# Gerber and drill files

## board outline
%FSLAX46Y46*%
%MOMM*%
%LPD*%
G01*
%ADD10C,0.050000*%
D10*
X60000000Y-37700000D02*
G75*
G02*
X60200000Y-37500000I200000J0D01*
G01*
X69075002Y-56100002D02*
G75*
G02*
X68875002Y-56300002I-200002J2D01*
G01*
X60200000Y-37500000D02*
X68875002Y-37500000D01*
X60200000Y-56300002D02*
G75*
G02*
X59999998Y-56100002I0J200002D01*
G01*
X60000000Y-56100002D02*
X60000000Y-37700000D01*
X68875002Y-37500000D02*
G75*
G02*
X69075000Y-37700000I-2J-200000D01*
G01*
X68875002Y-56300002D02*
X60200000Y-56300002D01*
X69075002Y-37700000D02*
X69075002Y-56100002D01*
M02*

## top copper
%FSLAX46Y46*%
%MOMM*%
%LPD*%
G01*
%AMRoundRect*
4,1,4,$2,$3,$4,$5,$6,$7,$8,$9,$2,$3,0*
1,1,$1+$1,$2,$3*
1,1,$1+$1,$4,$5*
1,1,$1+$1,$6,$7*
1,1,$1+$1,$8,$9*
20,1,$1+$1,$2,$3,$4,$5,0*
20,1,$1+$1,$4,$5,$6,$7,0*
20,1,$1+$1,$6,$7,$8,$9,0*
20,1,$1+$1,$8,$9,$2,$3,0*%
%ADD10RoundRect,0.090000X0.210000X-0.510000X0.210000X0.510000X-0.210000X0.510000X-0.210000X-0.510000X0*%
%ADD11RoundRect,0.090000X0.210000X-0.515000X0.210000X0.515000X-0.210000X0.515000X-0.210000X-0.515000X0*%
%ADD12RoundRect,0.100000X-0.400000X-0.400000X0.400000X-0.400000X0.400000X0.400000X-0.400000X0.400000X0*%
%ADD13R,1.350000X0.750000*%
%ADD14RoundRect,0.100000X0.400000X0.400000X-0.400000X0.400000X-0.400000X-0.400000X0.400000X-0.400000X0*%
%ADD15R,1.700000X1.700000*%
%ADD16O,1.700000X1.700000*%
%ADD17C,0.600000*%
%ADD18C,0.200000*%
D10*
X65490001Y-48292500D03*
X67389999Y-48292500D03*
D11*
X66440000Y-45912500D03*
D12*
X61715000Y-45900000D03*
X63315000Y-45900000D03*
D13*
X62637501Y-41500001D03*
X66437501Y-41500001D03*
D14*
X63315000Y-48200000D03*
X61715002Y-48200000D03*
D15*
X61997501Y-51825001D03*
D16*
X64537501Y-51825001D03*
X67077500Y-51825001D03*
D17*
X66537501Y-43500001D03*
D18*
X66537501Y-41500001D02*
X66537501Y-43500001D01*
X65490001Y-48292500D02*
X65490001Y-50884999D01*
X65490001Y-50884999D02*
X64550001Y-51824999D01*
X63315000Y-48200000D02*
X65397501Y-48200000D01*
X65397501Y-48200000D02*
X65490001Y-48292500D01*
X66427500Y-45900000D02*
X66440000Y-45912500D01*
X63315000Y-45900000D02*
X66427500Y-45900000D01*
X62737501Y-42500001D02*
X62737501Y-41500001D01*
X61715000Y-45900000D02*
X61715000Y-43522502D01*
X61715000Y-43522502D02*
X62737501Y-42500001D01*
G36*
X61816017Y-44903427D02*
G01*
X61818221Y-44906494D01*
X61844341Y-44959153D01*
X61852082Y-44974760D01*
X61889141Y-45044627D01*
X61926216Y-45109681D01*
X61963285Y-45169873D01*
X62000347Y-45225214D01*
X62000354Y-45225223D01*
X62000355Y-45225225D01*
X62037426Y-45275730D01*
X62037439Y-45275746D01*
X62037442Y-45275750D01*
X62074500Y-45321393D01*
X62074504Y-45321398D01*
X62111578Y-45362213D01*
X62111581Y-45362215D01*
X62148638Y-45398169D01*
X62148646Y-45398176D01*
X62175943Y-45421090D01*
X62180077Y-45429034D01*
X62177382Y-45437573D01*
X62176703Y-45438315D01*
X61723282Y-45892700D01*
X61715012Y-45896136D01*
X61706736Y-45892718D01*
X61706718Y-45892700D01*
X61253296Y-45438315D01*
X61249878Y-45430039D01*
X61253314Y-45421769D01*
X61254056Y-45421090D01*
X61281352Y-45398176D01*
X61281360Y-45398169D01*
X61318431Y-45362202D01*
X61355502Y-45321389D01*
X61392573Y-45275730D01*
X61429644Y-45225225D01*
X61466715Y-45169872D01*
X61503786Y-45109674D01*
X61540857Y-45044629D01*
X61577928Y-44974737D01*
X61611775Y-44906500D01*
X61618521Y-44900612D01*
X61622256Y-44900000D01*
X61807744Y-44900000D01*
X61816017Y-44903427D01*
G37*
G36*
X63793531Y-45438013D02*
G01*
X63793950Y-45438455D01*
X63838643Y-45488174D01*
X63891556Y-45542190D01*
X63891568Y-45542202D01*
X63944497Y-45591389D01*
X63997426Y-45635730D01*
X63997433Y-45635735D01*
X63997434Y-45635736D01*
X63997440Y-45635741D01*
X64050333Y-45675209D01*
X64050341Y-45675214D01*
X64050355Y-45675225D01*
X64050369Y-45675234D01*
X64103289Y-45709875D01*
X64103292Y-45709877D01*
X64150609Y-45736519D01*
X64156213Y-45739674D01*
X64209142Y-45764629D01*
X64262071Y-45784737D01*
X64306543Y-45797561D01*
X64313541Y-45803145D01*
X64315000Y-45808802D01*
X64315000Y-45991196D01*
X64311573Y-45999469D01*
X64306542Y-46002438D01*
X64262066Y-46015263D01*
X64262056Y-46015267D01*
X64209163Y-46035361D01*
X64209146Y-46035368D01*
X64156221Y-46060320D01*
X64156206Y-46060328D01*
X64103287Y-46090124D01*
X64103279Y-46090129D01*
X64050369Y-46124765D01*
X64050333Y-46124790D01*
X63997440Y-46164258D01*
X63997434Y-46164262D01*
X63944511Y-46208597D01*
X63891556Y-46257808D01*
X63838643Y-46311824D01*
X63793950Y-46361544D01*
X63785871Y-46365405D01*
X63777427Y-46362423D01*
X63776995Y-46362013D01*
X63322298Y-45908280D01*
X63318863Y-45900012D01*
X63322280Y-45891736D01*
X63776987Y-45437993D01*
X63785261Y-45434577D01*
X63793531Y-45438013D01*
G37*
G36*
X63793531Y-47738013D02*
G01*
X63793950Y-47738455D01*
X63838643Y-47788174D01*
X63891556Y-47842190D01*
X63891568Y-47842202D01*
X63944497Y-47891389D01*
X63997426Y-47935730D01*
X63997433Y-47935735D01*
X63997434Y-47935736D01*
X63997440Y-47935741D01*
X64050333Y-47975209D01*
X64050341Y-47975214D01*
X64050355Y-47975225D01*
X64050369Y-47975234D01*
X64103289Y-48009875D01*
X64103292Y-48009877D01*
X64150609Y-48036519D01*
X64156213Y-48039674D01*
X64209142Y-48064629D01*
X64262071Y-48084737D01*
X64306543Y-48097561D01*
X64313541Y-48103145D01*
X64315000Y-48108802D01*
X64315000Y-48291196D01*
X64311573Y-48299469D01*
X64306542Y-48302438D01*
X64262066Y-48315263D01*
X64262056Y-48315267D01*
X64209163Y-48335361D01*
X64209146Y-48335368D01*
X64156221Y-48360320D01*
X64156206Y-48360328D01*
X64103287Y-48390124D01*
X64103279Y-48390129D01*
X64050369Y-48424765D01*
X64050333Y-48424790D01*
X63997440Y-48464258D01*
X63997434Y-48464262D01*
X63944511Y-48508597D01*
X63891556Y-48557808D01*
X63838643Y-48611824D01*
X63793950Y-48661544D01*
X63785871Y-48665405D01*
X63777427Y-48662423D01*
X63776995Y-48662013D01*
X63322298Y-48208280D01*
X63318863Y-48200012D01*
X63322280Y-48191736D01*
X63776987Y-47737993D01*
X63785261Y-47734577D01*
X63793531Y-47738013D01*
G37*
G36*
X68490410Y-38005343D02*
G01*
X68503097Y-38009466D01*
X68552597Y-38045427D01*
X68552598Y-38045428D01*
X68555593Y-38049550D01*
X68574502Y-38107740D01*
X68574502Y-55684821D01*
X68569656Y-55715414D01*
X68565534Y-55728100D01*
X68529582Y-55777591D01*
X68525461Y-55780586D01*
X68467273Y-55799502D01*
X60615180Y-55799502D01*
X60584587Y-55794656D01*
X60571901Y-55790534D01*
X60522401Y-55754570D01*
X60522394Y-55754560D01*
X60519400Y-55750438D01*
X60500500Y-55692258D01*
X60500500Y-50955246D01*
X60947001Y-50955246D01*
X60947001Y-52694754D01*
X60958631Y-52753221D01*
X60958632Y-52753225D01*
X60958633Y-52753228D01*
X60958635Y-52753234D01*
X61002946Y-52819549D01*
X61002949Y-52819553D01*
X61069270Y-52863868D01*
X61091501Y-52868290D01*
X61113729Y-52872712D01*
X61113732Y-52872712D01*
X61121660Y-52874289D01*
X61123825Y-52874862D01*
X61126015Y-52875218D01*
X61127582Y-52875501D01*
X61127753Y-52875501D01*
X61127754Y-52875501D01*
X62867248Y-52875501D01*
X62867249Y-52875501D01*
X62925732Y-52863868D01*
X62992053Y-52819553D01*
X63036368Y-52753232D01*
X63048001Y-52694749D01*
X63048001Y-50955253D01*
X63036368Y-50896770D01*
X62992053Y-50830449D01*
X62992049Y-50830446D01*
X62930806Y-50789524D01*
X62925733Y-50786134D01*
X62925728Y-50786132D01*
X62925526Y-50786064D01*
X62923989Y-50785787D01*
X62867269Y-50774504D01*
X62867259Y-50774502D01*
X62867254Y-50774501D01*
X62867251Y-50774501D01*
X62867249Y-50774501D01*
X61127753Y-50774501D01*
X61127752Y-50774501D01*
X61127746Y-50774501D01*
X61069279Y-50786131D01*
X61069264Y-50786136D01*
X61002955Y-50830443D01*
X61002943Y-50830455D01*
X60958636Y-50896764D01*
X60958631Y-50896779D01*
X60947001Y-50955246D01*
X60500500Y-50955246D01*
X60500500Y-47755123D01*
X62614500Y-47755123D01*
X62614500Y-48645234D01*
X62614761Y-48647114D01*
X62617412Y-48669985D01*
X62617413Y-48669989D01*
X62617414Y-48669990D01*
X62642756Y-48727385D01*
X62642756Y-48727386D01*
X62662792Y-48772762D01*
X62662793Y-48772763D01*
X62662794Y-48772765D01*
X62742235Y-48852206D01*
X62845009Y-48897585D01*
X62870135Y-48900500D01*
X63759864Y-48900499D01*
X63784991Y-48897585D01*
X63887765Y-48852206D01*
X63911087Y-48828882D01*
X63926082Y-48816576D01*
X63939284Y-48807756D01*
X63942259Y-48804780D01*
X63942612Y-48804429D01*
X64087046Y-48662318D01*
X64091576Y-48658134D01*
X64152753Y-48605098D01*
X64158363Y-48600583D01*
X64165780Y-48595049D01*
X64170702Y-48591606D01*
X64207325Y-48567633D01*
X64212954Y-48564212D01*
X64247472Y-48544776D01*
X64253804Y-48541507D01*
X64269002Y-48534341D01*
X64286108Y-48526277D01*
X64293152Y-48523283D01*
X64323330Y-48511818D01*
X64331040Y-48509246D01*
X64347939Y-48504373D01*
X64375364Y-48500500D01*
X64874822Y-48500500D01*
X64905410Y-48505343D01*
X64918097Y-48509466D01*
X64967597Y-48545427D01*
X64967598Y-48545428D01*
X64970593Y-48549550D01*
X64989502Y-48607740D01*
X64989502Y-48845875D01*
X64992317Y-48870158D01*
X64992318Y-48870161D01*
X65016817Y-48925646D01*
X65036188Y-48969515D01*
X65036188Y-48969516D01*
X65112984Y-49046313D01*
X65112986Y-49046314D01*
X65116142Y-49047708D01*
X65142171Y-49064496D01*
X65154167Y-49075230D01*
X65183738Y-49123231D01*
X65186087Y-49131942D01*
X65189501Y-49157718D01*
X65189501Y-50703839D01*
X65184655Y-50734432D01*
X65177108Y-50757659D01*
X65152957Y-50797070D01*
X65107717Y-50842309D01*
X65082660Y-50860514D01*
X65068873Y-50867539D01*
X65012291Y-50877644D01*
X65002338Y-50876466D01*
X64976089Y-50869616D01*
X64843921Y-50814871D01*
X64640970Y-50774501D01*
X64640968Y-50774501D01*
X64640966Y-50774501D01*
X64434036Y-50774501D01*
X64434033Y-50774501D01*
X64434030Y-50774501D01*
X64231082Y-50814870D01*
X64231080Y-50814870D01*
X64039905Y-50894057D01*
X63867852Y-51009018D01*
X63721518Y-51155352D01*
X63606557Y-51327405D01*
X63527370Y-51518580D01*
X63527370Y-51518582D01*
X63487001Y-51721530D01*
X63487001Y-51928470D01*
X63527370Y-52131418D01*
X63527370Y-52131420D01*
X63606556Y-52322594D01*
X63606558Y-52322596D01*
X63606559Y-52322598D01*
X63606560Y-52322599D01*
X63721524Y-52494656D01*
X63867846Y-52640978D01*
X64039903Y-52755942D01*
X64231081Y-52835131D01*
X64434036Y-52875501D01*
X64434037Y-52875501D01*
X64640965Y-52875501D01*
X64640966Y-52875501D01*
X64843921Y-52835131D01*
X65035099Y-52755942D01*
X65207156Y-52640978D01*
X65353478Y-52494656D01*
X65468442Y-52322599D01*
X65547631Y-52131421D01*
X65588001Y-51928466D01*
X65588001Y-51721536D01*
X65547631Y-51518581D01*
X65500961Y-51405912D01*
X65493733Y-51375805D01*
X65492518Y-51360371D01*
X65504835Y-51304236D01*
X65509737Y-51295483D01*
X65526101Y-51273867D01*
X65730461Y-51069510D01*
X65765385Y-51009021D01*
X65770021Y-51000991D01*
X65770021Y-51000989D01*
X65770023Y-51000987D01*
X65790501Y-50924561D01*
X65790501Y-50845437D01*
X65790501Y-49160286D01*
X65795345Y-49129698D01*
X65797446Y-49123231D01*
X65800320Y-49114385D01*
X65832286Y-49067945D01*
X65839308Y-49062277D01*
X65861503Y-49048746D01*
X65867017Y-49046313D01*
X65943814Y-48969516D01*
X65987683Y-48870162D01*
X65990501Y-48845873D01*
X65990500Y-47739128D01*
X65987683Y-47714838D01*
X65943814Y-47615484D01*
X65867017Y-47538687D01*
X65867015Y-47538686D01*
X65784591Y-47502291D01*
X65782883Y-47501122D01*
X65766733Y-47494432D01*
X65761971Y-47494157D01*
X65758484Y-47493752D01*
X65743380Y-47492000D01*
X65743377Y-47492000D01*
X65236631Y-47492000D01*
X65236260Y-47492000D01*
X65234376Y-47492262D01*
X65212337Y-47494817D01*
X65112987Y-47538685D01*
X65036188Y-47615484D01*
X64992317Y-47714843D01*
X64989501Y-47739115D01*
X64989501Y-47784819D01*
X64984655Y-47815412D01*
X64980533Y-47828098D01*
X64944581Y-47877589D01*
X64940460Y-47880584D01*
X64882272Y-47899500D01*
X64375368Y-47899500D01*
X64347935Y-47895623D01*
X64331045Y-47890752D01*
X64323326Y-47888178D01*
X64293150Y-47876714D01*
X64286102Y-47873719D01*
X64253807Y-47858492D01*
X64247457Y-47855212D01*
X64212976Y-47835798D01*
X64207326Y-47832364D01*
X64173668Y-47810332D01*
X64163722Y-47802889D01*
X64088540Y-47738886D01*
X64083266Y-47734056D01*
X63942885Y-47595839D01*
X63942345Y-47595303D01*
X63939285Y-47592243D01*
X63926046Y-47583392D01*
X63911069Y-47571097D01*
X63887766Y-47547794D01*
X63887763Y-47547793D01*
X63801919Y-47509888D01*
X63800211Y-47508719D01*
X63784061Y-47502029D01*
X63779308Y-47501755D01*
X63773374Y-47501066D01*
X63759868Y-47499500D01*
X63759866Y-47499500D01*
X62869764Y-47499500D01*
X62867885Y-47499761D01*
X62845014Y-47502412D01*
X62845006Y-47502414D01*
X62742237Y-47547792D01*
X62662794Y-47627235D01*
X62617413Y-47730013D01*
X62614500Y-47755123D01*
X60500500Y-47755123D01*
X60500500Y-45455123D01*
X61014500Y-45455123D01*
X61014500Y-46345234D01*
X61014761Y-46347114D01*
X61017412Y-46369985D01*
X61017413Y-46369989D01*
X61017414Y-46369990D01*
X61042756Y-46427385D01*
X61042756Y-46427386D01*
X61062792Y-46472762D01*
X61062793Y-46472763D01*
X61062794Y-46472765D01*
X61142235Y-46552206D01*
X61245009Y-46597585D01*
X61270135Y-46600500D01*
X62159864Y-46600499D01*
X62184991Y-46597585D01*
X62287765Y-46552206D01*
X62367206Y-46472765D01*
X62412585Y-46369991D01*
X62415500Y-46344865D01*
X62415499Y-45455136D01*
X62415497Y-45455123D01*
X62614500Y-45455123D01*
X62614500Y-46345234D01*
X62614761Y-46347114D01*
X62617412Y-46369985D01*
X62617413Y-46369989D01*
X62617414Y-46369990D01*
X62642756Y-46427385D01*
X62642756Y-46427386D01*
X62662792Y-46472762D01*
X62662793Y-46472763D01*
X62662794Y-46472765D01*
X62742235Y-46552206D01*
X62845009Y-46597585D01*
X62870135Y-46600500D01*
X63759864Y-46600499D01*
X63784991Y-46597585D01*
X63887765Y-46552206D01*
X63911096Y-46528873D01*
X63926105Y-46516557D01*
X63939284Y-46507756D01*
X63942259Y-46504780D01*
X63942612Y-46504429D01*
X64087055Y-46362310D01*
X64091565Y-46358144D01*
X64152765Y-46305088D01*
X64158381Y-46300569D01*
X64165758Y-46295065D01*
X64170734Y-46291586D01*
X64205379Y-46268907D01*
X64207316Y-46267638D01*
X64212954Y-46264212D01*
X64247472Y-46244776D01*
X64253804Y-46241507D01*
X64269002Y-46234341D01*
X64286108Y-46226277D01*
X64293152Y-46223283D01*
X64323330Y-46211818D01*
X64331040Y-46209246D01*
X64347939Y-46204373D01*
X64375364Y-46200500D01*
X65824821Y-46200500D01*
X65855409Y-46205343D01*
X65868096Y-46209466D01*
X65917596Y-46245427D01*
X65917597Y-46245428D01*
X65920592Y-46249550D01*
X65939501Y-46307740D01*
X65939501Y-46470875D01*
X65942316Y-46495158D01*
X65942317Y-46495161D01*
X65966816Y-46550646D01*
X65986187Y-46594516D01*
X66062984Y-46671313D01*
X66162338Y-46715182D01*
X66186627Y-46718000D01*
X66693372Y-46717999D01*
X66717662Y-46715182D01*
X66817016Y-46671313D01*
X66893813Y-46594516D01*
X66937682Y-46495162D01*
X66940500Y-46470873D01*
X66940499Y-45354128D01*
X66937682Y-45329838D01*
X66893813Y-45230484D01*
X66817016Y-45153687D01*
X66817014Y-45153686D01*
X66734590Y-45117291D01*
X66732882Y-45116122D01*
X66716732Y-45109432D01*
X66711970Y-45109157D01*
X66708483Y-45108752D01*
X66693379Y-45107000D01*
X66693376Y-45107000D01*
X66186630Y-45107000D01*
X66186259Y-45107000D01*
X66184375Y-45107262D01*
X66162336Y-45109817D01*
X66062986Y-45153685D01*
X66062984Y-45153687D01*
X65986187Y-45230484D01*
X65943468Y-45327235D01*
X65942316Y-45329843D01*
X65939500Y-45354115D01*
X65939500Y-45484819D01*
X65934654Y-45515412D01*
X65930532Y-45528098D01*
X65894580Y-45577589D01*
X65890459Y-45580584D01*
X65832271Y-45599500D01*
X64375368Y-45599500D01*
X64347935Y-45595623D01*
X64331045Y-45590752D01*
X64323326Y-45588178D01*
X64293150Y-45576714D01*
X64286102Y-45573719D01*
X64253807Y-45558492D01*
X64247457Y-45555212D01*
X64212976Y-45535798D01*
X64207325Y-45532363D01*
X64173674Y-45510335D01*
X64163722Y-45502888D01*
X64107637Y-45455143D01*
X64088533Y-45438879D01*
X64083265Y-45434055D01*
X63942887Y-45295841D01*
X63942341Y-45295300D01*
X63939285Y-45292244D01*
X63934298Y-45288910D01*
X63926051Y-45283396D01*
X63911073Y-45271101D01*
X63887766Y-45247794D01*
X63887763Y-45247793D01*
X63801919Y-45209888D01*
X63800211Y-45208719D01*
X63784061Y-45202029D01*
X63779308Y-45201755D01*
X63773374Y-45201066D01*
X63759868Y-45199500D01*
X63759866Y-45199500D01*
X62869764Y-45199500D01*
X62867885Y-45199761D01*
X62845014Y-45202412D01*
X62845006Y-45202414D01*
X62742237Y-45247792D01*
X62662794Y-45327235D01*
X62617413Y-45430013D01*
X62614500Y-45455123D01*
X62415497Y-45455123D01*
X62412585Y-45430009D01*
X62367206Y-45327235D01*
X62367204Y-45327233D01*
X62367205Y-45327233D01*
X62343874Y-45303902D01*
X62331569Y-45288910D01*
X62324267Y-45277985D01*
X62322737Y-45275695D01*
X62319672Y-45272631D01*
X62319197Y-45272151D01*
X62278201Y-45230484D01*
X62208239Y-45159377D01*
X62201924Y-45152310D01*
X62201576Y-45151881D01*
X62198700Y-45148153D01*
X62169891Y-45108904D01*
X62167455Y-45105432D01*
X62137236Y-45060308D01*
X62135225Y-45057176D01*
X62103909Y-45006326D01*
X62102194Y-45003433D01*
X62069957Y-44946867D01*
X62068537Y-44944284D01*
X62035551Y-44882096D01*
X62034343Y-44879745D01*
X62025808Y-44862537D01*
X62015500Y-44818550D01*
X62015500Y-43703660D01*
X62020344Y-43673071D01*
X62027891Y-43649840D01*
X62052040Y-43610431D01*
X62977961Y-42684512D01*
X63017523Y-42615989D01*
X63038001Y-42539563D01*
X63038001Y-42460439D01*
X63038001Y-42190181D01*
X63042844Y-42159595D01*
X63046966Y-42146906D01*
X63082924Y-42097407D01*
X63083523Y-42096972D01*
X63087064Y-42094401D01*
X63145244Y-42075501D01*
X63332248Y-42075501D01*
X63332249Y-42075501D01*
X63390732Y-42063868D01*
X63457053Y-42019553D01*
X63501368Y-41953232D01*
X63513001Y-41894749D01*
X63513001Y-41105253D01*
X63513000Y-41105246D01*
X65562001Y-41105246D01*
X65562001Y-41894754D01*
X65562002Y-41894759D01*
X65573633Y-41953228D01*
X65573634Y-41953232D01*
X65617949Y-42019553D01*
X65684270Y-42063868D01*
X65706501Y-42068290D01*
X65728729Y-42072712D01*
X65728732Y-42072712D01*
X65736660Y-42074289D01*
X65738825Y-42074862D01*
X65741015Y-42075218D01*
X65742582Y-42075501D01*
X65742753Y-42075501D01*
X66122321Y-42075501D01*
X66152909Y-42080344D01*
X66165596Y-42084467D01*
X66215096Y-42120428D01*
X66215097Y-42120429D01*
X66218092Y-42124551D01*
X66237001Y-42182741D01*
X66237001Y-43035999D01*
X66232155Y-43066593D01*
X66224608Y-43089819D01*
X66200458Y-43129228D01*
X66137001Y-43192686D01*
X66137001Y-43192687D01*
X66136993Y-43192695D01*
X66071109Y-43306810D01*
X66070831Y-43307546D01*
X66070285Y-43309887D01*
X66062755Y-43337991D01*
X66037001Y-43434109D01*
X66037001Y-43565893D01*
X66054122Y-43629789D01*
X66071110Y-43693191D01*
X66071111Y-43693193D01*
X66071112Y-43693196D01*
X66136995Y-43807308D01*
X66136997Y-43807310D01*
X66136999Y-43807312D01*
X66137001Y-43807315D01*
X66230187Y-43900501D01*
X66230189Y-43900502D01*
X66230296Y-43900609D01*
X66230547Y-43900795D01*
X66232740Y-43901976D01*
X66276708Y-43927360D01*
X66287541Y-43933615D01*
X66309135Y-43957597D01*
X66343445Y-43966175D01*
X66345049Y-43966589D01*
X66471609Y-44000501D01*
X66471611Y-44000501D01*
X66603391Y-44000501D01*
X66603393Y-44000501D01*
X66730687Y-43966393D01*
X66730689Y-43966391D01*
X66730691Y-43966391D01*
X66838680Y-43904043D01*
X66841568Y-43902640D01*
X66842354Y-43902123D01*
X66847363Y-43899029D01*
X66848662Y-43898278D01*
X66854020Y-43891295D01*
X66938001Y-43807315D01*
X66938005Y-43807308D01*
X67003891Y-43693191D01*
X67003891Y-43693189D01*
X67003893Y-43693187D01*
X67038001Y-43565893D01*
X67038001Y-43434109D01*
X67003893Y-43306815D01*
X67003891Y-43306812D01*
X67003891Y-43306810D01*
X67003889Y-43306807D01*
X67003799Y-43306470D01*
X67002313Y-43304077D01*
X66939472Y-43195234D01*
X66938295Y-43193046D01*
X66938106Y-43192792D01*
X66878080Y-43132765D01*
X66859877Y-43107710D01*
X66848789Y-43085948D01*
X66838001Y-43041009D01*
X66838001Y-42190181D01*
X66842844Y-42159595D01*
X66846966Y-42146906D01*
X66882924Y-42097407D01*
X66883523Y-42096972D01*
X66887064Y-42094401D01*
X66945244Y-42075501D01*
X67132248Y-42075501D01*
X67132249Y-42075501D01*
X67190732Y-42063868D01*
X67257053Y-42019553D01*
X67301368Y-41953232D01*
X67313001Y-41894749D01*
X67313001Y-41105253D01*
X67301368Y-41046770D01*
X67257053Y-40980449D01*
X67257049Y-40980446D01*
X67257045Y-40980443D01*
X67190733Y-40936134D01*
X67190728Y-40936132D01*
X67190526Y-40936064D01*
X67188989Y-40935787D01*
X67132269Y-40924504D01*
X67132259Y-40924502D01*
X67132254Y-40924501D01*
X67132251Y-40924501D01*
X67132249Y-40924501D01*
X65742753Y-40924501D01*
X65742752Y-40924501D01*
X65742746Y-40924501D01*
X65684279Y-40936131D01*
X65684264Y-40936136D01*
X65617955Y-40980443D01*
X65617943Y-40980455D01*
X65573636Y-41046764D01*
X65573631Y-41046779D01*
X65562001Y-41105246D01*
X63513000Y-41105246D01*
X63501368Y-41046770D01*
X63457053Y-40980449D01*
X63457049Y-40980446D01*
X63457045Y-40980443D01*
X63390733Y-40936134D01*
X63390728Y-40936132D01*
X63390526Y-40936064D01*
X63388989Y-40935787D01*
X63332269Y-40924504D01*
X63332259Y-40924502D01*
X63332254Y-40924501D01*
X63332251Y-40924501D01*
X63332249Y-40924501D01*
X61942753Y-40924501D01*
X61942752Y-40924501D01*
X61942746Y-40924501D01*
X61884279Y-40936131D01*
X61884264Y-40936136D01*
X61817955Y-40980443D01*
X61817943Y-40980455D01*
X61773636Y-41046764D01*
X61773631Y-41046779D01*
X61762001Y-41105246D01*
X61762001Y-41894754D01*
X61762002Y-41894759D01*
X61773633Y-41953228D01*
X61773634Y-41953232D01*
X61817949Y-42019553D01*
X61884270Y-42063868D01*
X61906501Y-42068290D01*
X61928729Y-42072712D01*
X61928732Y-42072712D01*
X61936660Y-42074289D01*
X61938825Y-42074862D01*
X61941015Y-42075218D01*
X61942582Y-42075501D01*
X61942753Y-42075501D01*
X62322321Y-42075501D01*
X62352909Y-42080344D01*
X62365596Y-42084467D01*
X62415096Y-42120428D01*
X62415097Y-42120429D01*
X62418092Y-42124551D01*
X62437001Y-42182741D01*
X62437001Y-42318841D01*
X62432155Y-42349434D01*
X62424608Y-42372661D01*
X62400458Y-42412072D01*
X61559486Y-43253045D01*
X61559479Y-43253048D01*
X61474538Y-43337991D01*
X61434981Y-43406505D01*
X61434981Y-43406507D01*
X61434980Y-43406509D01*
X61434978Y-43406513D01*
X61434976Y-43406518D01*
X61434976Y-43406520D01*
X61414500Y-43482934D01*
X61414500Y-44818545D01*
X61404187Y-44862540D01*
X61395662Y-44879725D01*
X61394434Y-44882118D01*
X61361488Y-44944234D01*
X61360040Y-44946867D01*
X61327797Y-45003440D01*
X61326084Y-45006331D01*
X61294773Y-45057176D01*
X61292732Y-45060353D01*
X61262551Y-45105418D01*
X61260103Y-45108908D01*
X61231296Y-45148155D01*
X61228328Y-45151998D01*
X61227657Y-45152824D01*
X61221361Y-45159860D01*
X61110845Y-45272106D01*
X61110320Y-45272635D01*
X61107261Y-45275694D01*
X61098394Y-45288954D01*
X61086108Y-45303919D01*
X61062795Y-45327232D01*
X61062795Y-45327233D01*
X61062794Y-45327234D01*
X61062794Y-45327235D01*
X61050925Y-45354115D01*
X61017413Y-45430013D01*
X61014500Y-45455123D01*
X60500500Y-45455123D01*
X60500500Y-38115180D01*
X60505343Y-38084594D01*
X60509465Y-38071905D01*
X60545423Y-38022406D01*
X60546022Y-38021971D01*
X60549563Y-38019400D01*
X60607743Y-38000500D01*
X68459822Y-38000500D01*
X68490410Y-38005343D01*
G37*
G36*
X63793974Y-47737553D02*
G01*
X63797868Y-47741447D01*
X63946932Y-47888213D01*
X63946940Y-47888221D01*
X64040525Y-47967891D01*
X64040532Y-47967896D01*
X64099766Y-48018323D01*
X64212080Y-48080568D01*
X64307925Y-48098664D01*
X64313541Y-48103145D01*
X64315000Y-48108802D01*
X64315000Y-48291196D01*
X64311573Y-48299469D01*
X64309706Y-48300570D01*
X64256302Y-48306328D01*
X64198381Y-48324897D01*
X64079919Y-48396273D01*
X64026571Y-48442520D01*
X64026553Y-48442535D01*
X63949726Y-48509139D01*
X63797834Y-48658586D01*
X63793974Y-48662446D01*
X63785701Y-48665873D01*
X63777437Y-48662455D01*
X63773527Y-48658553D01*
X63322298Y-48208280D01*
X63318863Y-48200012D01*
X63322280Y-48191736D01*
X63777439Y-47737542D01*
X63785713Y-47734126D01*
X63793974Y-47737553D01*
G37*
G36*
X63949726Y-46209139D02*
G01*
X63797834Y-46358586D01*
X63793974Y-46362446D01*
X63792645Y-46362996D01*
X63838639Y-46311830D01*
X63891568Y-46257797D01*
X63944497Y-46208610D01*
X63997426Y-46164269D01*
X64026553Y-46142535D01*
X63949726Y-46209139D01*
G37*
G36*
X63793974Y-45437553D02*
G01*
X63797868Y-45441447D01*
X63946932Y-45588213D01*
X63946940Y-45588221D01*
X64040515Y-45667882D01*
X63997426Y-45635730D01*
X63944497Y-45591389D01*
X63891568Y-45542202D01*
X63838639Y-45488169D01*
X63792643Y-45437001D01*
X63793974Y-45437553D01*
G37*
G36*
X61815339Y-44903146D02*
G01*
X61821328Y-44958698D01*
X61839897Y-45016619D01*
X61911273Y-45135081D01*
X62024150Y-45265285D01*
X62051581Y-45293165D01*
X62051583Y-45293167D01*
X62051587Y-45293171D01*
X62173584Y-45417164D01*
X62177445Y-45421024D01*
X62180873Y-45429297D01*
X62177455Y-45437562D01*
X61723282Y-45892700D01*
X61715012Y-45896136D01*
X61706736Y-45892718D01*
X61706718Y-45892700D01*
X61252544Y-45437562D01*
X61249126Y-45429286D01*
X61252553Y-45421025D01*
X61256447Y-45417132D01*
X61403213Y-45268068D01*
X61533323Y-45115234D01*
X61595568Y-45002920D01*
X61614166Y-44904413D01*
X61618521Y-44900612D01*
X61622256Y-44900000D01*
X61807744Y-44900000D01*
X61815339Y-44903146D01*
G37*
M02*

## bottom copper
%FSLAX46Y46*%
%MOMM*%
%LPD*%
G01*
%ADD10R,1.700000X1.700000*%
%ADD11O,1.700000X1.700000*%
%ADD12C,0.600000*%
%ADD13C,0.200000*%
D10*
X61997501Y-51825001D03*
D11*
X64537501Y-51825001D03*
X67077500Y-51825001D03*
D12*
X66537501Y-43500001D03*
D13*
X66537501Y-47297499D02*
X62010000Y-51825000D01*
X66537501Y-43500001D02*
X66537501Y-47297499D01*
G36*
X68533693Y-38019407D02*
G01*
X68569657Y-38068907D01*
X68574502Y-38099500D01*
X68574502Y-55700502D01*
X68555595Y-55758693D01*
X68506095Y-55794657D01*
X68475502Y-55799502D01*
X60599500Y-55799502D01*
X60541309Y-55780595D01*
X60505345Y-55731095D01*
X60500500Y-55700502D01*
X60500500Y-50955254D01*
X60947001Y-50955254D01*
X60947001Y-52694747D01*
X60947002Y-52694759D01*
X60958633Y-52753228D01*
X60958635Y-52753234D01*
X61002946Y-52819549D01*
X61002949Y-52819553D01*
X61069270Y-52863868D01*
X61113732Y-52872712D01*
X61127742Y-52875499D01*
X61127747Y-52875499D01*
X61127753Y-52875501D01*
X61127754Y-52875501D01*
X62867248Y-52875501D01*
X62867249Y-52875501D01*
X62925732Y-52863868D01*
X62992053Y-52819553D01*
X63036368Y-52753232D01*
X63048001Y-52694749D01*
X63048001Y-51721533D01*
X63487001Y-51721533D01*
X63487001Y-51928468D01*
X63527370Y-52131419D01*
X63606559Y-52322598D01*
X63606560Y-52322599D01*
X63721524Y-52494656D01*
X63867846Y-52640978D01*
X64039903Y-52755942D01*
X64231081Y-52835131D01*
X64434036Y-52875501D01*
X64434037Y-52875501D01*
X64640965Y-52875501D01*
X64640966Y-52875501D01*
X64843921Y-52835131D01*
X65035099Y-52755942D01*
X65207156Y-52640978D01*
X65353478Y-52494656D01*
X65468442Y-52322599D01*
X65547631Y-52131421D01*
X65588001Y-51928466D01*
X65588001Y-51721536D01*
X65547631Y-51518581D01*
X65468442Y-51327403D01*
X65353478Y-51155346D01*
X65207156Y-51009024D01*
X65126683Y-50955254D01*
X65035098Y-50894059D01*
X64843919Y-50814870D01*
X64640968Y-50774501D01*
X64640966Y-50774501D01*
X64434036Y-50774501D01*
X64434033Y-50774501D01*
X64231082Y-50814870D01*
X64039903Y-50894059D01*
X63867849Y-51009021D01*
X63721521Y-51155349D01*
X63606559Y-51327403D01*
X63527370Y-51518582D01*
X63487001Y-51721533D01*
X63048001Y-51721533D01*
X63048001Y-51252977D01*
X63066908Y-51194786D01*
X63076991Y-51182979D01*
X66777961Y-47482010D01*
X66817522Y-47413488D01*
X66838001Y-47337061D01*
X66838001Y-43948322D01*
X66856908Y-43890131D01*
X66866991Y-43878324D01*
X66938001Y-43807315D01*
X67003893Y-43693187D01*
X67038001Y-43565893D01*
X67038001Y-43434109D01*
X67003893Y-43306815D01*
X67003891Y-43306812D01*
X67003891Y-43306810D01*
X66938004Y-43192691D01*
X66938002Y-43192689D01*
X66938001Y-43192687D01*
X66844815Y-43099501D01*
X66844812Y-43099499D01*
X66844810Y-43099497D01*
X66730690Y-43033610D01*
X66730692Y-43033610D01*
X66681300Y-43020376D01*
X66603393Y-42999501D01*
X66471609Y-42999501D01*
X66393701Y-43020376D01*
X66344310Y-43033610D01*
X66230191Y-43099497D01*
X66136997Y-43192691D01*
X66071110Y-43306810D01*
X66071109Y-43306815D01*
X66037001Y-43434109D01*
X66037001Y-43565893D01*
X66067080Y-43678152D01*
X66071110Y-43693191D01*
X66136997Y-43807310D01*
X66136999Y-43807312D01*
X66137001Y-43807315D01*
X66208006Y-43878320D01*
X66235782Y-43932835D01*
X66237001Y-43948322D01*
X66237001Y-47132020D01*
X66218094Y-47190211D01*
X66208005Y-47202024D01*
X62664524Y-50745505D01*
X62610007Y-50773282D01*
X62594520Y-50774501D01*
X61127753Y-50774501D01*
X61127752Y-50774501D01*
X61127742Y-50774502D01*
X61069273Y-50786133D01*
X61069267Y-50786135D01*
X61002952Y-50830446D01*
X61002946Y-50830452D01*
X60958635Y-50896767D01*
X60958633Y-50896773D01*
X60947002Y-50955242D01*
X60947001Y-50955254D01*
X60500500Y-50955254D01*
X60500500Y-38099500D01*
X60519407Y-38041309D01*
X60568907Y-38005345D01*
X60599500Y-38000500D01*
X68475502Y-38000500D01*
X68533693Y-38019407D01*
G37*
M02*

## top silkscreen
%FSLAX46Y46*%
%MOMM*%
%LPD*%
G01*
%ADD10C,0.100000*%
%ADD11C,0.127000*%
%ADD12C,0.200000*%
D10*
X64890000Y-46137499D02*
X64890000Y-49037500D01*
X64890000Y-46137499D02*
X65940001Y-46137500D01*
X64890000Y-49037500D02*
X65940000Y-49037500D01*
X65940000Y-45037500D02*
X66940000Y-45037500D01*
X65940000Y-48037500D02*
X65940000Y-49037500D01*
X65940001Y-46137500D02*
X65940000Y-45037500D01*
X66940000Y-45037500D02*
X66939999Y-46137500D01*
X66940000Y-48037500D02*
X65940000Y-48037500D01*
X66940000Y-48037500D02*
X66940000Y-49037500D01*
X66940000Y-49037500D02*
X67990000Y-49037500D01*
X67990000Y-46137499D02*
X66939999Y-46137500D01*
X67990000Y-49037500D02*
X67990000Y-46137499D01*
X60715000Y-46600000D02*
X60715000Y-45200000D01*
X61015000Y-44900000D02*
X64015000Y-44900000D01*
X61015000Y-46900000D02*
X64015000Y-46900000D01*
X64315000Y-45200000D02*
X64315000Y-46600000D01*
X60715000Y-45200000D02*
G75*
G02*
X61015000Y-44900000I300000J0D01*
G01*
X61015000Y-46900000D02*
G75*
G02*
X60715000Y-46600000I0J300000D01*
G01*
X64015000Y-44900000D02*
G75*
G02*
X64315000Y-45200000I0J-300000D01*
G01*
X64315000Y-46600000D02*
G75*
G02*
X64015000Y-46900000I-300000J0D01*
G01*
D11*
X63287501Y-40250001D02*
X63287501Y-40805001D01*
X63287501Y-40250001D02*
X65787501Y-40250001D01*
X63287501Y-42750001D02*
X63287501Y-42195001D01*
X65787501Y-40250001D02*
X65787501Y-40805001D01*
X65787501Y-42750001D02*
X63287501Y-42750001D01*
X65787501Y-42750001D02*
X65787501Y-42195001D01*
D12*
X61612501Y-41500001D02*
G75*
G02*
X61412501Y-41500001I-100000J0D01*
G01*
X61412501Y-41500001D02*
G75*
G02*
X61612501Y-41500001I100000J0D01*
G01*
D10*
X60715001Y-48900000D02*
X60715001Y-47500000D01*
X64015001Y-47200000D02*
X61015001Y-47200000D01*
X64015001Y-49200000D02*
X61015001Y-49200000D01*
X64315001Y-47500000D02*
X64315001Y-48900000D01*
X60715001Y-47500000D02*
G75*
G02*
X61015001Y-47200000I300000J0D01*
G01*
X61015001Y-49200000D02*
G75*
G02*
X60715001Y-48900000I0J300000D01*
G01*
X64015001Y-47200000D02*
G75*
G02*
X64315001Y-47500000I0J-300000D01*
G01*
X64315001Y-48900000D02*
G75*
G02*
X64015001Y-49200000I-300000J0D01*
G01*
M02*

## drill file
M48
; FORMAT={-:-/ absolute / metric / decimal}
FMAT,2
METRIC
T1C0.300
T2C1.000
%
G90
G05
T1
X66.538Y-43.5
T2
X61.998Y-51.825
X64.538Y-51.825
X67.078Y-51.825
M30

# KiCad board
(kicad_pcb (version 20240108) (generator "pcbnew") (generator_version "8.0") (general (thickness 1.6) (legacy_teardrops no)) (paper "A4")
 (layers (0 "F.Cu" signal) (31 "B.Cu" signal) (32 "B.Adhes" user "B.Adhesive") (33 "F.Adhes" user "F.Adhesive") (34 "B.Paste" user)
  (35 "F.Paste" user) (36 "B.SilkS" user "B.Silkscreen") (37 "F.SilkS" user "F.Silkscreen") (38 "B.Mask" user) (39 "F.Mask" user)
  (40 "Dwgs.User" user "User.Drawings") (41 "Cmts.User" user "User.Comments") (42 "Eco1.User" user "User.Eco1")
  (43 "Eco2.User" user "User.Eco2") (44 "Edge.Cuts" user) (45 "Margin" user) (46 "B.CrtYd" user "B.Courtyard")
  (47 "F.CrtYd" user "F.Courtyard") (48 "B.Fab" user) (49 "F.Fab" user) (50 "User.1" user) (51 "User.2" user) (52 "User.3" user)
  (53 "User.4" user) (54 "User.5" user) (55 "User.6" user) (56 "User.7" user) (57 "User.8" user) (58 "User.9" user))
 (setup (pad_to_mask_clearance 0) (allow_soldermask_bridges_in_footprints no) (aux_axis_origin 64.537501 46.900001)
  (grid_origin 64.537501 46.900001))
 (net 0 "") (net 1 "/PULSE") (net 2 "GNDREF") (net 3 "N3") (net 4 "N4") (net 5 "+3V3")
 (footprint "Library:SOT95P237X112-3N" (layer "F.Cu") (at 66.44 47.0375 90)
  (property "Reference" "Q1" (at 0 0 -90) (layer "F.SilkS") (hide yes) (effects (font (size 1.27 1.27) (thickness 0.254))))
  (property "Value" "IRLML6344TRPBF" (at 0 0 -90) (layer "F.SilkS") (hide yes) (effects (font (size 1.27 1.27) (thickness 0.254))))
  (fp_line (start 0.900001 -1.55) (end -2 -1.55) (stroke (width 0.1) (type solid)) (layer "F.SilkS"))
  (fp_line (start 0.900001 -1.55) (end 0.9 -0.499999) (stroke (width 0.1) (type default)) (layer "F.SilkS"))
  (fp_line (start -2 -1.55) (end -2 -0.5) (stroke (width 0.1) (type default)) (layer "F.SilkS"))
  (fp_line (start 2 -0.5) (end 2 0.5) (stroke (width 0.1) (type default)) (layer "F.SilkS"))
  (fp_line (start -1 -0.5) (end -2 -0.5) (stroke (width 0.1) (type default)) (layer "F.SilkS"))
  (fp_line (start 0.9 -0.499999) (end 2 -0.5) (stroke (width 0.1) (type default)) (layer "F.SilkS"))
  (fp_line (start 2 0.5) (end 0.9 0.499999) (stroke (width 0.1) (type default)) (layer "F.SilkS"))
  (fp_line (start -1 0.5) (end -1 -0.5) (stroke (width 0.1) (type default)) (layer "F.SilkS"))
  (fp_line (start -1 0.5) (end -2 0.5) (stroke (width 0.1) (type default)) (layer "F.SilkS"))
  (fp_line (start -2 0.5) (end -2 1.55) (stroke (width 0.1) (type default)) (layer "F.SilkS"))
  (fp_line (start 0.900001 1.55) (end 0.9 0.499999) (stroke (width 0.1) (type default)) (layer "F.SilkS"))
  (fp_line (start -2 1.55) (end 0.900001 1.55) (stroke (width 0.1) (type solid)) (layer "F.SilkS"))
  (pad "1" smd roundrect (at -1.255 -0.949999 90) (size 1.2 0.6) (layers "F.Cu" "F.Paste" "F.Mask") (roundrect_rratio 0.15) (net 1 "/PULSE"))
  (pad "2" smd roundrect (at -1.255 0.949999 90) (size 1.2 0.6) (layers "F.Cu" "F.Paste" "F.Mask") (roundrect_rratio 0.15) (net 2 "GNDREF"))
  (pad "3" smd roundrect (at 1.125 0 90) (size 1.21 0.6) (layers "F.Cu" "F.Paste" "F.Mask") (roundrect_rratio 0.15) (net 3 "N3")))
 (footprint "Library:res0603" (layer "F.Cu") (at 62.515 45.9)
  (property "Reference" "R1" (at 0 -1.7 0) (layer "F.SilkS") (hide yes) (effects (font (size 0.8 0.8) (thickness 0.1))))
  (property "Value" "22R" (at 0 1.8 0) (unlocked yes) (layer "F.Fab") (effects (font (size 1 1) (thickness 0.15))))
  (fp_line (start -1.8 0.7) (end -1.8 -0.7) (stroke (width 0.1) (type default)) (layer "F.SilkS"))
  (fp_line (start -1.5 -1) (end 1.5 -1) (stroke (width 0.1) (type default)) (layer "F.SilkS"))
  (fp_line (start -1.5 1) (end 1.5 1) (stroke (width 0.1) (type default)) (layer "F.SilkS"))
  (fp_line (start 1.8 -0.7) (end 1.8 0.7) (stroke (width 0.1) (type default)) (layer "F.SilkS"))
  (fp_arc (start -1.8 -0.7) (mid -1.712132 -0.912132) (end -1.5 -1) (stroke (width 0.1) (type default)) (layer "F.SilkS"))
  (fp_arc (start -1.5 1) (mid -1.712132 0.912132) (end -1.8 0.7) (stroke (width 0.1) (type default)) (layer "F.SilkS"))
  (fp_arc (start 1.5 -1) (mid 1.712132 -0.912132) (end 1.8 -0.7) (stroke (width 0.1) (type default)) (layer "F.SilkS"))
  (fp_arc (start 1.8 0.7) (mid 1.712132 0.912132) (end 1.5 1) (stroke (width 0.1) (type default)) (layer "F.SilkS"))
  (pad "1" smd roundrect (at -0.8 0) (size 1 1) (layers "F.Cu" "F.Paste" "F.Mask") (roundrect_rratio 0.1) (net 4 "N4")
   (thermal_bridge_angle 45)
   (teardrops (best_length_ratio 0.5) (max_length 1) (best_width_ratio 1) (max_width 1) (curve_points 10) (filter_ratio 0.9) (enabled yes)
    (allow_two_segments yes) (prefer_zone_connections yes)))
  (pad "2" smd roundrect (at 0.8 0) (size 1 1) (layers "F.Cu" "F.Paste" "F.Mask") (roundrect_rratio 0.1) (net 3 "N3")
   (thermal_bridge_angle 45)
   (teardrops (best_length_ratio 0.5) (max_length 1) (best_width_ratio 1) (max_width 1) (curve_points 10) (filter_ratio 0.9) (enabled yes)
    (allow_two_segments yes) (prefer_zone_connections yes))))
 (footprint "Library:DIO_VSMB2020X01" (layer "F.Cu") (at 64.537501 41.500001)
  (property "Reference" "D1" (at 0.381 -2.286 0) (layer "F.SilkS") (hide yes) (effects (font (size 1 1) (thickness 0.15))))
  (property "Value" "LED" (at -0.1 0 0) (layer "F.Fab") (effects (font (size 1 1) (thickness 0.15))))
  (fp_line (start -1.25 -1.25) (end -1.25 -0.695) (stroke (width 0.127) (type solid)) (layer "F.SilkS"))
  (fp_line (start -1.25 -1.25) (end 1.25 -1.25) (stroke (width 0.127) (type solid)) (layer "F.SilkS"))
  (fp_line (start -1.25 1.25) (end -1.25 0.695) (stroke (width 0.127) (type solid)) (layer "F.SilkS"))
  (fp_line (start 1.25 -1.25) (end 1.25 -0.695) (stroke (width 0.127) (type solid)) (layer "F.SilkS"))
  (fp_line (start 1.25 1.25) (end -1.25 1.25) (stroke (width 0.127) (type solid)) (layer "F.SilkS"))
  (fp_line (start 1.25 1.25) (end 1.25 0.695) (stroke (width 0.127) (type solid)) (layer "F.SilkS"))
  (fp_circle (center -3.025 0) (end -2.925 0) (stroke (width 0.2) (type solid)) (fill none) (layer "F.SilkS"))
  (pad "1" smd rect (at -1.9 0) (size 1.35 0.75) (layers "F.Cu" "F.Paste" "F.Mask") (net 4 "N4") (solder_mask_margin 0.102))
  (pad "2" smd rect (at 1.9 0) (size 1.35 0.75) (layers "F.Cu" "F.Paste" "F.Mask") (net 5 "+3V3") (solder_mask_margin 0.102)))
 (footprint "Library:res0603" (layer "F.Cu") (at 62.515001 48.2 180)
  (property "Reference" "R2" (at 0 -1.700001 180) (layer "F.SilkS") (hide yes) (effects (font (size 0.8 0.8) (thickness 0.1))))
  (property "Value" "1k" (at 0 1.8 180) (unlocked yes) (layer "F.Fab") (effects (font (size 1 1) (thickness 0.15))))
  (fp_line (start 1.8 -0.7) (end 1.8 0.7) (stroke (width 0.1) (type default)) (layer "F.SilkS"))
  (fp_line (start -1.5 1) (end 1.5 1) (stroke (width 0.1) (type default)) (layer "F.SilkS"))
  (fp_line (start -1.5 -1) (end 1.5 -1) (stroke (width 0.1) (type default)) (layer "F.SilkS"))
  (fp_line (start -1.8 0.7) (end -1.8 -0.7) (stroke (width 0.1) (type default)) (layer "F.SilkS"))
  (fp_arc (start 1.8 0.7) (mid 1.712132 0.912132) (end 1.5 1) (stroke (width 0.1) (type default)) (layer "F.SilkS"))
  (fp_arc (start 1.5 -1) (mid 1.712132 -0.912132) (end 1.8 -0.7) (stroke (width 0.1) (type default)) (layer "F.SilkS"))
  (fp_arc (start -1.5 1) (mid -1.712132 0.912132) (end -1.8 0.7) (stroke (width 0.1) (type default)) (layer "F.SilkS"))
  (fp_arc (start -1.8 -0.7) (mid -1.712132 -0.912132) (end -1.5 -1) (stroke (width 0.1) (type default)) (layer "F.SilkS"))
  (pad "1" smd roundrect (at -0.799999 0 180) (size 1 1) (layers "F.Cu" "F.Paste" "F.Mask") (roundrect_rratio 0.1) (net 1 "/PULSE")
   (thermal_bridge_angle 45)
   (teardrops (best_length_ratio 0.5) (max_length 1) (best_width_ratio 1) (max_width 1) (curve_points 10) (filter_ratio 0.9) (enabled yes)
    (allow_two_segments yes) (prefer_zone_connections yes)))
  (pad "2" smd roundrect (at 0.799999 0 180) (size 1 1) (layers "F.Cu" "F.Paste" "F.Mask") (roundrect_rratio 0.1) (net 2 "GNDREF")
   (thermal_bridge_angle 45)
   (teardrops (best_length_ratio 0.5) (max_length 1) (best_width_ratio 1) (max_width 1) (curve_points 10) (filter_ratio 0.9) (enabled yes)
    (allow_two_segments yes) (prefer_zone_connections yes))))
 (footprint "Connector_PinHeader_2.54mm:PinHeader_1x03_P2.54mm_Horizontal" (layer "B.Cu") (at 61.997501 51.825001 -90)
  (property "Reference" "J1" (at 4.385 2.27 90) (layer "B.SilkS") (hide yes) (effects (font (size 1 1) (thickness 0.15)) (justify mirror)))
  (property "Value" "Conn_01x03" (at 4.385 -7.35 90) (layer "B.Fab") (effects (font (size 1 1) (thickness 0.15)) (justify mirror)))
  (pad "1" thru_hole rect (at 0 0 270) (size 1.7 1.7) (drill 1) (layers "*.Cu" "*.Mask") (remove_unused_layers no) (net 5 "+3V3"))
  (pad "2" thru_hole oval (at 0 -2.54 270) (size 1.7 1.7) (drill 1) (layers "*.Cu" "*.Mask") (remove_unused_layers no) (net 1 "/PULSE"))
  (pad "3" thru_hole oval (at 0 -5.079999 270) (size 1.7 1.7) (drill 1) (layers "*.Cu" "*.Mask") (remove_unused_layers no) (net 2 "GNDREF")))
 (gr_arc (start 60 37.7) (mid 60.058579 37.558579) (end 60.2 37.5) (stroke (width 0.05) (type default)) (layer "Edge.Cuts"))
 (gr_arc (start 69.075002 56.100002) (mid 69.016423 56.241423) (end 68.875002 56.300002) (stroke (width 0.05) (type default))
  (layer "Edge.Cuts"))
 (gr_line (start 60.2 37.5) (end 68.875002 37.5) (stroke (width 0.05) (type default)) (layer "Edge.Cuts"))
 (gr_arc (start 60.2 56.300002) (mid 60.058579 56.241423) (end 60 56.100002) (stroke (width 0.05) (type default)) (layer "Edge.Cuts"))
 (gr_line (start 60 56.100002) (end 60 37.7) (stroke (width 0.05) (type default)) (layer "Edge.Cuts"))
 (gr_arc (start 68.875002 37.5) (mid 69.016423 37.558579) (end 69.075002 37.7) (stroke (width 0.05) (type default)) (layer "Edge.Cuts"))
 (gr_line (start 68.875002 56.300002) (end 60.2 56.300002) (stroke (width 0.05) (type default)) (layer "Edge.Cuts"))
 (gr_line (start 69.075002 37.7) (end 69.075002 56.100002) (stroke (width 0.05) (type default)) (layer "Edge.Cuts"))
 (segment (start 66.537501 41.500001) (end 66.537501 43.500001) (width 0.2) (layer "F.Cu") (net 5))
 (via (at 66.537501 43.500001) (size 0.6) (drill 0.3) (layers "F.Cu" "B.Cu") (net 5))
 (segment (start 66.537501 47.297499) (end 62.01 51.825) (width 0.2) (layer "B.Cu") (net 5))
 (segment (start 66.537501 43.500001) (end 66.537501 47.297499) (width 0.2) (layer "B.Cu") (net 5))
 (segment (start 65.490001 48.2925) (end 65.490001 50.884999) (width 0.2) (layer "F.Cu") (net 1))
 (segment (start 65.490001 50.884999) (end 64.550001 51.824999) (width 0.2) (layer "F.Cu") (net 1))
 (segment (start 63.315 48.2) (end 65.397501 48.2) (width 0.2) (layer "F.Cu") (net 1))
 (segment (start 65.397501 48.2) (end 65.490001 48.2925) (width 0.2) (layer "F.Cu") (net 1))
 (segment (start 66.4275 45.9) (end 66.44 45.9125) (width 0.2) (layer "F.Cu") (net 3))
 (segment (start 63.315 45.9) (end 66.4275 45.9) (width 0.2) (layer "F.Cu") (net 3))
 (segment (start 62.737501 42.500001) (end 62.737501 41.500001) (width 0.2) (layer "F.Cu") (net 4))
 (segment (start 61.715 45.9) (end 61.715 43.522502) (width 0.2) (layer "F.Cu") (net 4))
 (segment (start 61.715 43.522502) (end 62.737501 42.500001) (width 0.2) (layer "F.Cu") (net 4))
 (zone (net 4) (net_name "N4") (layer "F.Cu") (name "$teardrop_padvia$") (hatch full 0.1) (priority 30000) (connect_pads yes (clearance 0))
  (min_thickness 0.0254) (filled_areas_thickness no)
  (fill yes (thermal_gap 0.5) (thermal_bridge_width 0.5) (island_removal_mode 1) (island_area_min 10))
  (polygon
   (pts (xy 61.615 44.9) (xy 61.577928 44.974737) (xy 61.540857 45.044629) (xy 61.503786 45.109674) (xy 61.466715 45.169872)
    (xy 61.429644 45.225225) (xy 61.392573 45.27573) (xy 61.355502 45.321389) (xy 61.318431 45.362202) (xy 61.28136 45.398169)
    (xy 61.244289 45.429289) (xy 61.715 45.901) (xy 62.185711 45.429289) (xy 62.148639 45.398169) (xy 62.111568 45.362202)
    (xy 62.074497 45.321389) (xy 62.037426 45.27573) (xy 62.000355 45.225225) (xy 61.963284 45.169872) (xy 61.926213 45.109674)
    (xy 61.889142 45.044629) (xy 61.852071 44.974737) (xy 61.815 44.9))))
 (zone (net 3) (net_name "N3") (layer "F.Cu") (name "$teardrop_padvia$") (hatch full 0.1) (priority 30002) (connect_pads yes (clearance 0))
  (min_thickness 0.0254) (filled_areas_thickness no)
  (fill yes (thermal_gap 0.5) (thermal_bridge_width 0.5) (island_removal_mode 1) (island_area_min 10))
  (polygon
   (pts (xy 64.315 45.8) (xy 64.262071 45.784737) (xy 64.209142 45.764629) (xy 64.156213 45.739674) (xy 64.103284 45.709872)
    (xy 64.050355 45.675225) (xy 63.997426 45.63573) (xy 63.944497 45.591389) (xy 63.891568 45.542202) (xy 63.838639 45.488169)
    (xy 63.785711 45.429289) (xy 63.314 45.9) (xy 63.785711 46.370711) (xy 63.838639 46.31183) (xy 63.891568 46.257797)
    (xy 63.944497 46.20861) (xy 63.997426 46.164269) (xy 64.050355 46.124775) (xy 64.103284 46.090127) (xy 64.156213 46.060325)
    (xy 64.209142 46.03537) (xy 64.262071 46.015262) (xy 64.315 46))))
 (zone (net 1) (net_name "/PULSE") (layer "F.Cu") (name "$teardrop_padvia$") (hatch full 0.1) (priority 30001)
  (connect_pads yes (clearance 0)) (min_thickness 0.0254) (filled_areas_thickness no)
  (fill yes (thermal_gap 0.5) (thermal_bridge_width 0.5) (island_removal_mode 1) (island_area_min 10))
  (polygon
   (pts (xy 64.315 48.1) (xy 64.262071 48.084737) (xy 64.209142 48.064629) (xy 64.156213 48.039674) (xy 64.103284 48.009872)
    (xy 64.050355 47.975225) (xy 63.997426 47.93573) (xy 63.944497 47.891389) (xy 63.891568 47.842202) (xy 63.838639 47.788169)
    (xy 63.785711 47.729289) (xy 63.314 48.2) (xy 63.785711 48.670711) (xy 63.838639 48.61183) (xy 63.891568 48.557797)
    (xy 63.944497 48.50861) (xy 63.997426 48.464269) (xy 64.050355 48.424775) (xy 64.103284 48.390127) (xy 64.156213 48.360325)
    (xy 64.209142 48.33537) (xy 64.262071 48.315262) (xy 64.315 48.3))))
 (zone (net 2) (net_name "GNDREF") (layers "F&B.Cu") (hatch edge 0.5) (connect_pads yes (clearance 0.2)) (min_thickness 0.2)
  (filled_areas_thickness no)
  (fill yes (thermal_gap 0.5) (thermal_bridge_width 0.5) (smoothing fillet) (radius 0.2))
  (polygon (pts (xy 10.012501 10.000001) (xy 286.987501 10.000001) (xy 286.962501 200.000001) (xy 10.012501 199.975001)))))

